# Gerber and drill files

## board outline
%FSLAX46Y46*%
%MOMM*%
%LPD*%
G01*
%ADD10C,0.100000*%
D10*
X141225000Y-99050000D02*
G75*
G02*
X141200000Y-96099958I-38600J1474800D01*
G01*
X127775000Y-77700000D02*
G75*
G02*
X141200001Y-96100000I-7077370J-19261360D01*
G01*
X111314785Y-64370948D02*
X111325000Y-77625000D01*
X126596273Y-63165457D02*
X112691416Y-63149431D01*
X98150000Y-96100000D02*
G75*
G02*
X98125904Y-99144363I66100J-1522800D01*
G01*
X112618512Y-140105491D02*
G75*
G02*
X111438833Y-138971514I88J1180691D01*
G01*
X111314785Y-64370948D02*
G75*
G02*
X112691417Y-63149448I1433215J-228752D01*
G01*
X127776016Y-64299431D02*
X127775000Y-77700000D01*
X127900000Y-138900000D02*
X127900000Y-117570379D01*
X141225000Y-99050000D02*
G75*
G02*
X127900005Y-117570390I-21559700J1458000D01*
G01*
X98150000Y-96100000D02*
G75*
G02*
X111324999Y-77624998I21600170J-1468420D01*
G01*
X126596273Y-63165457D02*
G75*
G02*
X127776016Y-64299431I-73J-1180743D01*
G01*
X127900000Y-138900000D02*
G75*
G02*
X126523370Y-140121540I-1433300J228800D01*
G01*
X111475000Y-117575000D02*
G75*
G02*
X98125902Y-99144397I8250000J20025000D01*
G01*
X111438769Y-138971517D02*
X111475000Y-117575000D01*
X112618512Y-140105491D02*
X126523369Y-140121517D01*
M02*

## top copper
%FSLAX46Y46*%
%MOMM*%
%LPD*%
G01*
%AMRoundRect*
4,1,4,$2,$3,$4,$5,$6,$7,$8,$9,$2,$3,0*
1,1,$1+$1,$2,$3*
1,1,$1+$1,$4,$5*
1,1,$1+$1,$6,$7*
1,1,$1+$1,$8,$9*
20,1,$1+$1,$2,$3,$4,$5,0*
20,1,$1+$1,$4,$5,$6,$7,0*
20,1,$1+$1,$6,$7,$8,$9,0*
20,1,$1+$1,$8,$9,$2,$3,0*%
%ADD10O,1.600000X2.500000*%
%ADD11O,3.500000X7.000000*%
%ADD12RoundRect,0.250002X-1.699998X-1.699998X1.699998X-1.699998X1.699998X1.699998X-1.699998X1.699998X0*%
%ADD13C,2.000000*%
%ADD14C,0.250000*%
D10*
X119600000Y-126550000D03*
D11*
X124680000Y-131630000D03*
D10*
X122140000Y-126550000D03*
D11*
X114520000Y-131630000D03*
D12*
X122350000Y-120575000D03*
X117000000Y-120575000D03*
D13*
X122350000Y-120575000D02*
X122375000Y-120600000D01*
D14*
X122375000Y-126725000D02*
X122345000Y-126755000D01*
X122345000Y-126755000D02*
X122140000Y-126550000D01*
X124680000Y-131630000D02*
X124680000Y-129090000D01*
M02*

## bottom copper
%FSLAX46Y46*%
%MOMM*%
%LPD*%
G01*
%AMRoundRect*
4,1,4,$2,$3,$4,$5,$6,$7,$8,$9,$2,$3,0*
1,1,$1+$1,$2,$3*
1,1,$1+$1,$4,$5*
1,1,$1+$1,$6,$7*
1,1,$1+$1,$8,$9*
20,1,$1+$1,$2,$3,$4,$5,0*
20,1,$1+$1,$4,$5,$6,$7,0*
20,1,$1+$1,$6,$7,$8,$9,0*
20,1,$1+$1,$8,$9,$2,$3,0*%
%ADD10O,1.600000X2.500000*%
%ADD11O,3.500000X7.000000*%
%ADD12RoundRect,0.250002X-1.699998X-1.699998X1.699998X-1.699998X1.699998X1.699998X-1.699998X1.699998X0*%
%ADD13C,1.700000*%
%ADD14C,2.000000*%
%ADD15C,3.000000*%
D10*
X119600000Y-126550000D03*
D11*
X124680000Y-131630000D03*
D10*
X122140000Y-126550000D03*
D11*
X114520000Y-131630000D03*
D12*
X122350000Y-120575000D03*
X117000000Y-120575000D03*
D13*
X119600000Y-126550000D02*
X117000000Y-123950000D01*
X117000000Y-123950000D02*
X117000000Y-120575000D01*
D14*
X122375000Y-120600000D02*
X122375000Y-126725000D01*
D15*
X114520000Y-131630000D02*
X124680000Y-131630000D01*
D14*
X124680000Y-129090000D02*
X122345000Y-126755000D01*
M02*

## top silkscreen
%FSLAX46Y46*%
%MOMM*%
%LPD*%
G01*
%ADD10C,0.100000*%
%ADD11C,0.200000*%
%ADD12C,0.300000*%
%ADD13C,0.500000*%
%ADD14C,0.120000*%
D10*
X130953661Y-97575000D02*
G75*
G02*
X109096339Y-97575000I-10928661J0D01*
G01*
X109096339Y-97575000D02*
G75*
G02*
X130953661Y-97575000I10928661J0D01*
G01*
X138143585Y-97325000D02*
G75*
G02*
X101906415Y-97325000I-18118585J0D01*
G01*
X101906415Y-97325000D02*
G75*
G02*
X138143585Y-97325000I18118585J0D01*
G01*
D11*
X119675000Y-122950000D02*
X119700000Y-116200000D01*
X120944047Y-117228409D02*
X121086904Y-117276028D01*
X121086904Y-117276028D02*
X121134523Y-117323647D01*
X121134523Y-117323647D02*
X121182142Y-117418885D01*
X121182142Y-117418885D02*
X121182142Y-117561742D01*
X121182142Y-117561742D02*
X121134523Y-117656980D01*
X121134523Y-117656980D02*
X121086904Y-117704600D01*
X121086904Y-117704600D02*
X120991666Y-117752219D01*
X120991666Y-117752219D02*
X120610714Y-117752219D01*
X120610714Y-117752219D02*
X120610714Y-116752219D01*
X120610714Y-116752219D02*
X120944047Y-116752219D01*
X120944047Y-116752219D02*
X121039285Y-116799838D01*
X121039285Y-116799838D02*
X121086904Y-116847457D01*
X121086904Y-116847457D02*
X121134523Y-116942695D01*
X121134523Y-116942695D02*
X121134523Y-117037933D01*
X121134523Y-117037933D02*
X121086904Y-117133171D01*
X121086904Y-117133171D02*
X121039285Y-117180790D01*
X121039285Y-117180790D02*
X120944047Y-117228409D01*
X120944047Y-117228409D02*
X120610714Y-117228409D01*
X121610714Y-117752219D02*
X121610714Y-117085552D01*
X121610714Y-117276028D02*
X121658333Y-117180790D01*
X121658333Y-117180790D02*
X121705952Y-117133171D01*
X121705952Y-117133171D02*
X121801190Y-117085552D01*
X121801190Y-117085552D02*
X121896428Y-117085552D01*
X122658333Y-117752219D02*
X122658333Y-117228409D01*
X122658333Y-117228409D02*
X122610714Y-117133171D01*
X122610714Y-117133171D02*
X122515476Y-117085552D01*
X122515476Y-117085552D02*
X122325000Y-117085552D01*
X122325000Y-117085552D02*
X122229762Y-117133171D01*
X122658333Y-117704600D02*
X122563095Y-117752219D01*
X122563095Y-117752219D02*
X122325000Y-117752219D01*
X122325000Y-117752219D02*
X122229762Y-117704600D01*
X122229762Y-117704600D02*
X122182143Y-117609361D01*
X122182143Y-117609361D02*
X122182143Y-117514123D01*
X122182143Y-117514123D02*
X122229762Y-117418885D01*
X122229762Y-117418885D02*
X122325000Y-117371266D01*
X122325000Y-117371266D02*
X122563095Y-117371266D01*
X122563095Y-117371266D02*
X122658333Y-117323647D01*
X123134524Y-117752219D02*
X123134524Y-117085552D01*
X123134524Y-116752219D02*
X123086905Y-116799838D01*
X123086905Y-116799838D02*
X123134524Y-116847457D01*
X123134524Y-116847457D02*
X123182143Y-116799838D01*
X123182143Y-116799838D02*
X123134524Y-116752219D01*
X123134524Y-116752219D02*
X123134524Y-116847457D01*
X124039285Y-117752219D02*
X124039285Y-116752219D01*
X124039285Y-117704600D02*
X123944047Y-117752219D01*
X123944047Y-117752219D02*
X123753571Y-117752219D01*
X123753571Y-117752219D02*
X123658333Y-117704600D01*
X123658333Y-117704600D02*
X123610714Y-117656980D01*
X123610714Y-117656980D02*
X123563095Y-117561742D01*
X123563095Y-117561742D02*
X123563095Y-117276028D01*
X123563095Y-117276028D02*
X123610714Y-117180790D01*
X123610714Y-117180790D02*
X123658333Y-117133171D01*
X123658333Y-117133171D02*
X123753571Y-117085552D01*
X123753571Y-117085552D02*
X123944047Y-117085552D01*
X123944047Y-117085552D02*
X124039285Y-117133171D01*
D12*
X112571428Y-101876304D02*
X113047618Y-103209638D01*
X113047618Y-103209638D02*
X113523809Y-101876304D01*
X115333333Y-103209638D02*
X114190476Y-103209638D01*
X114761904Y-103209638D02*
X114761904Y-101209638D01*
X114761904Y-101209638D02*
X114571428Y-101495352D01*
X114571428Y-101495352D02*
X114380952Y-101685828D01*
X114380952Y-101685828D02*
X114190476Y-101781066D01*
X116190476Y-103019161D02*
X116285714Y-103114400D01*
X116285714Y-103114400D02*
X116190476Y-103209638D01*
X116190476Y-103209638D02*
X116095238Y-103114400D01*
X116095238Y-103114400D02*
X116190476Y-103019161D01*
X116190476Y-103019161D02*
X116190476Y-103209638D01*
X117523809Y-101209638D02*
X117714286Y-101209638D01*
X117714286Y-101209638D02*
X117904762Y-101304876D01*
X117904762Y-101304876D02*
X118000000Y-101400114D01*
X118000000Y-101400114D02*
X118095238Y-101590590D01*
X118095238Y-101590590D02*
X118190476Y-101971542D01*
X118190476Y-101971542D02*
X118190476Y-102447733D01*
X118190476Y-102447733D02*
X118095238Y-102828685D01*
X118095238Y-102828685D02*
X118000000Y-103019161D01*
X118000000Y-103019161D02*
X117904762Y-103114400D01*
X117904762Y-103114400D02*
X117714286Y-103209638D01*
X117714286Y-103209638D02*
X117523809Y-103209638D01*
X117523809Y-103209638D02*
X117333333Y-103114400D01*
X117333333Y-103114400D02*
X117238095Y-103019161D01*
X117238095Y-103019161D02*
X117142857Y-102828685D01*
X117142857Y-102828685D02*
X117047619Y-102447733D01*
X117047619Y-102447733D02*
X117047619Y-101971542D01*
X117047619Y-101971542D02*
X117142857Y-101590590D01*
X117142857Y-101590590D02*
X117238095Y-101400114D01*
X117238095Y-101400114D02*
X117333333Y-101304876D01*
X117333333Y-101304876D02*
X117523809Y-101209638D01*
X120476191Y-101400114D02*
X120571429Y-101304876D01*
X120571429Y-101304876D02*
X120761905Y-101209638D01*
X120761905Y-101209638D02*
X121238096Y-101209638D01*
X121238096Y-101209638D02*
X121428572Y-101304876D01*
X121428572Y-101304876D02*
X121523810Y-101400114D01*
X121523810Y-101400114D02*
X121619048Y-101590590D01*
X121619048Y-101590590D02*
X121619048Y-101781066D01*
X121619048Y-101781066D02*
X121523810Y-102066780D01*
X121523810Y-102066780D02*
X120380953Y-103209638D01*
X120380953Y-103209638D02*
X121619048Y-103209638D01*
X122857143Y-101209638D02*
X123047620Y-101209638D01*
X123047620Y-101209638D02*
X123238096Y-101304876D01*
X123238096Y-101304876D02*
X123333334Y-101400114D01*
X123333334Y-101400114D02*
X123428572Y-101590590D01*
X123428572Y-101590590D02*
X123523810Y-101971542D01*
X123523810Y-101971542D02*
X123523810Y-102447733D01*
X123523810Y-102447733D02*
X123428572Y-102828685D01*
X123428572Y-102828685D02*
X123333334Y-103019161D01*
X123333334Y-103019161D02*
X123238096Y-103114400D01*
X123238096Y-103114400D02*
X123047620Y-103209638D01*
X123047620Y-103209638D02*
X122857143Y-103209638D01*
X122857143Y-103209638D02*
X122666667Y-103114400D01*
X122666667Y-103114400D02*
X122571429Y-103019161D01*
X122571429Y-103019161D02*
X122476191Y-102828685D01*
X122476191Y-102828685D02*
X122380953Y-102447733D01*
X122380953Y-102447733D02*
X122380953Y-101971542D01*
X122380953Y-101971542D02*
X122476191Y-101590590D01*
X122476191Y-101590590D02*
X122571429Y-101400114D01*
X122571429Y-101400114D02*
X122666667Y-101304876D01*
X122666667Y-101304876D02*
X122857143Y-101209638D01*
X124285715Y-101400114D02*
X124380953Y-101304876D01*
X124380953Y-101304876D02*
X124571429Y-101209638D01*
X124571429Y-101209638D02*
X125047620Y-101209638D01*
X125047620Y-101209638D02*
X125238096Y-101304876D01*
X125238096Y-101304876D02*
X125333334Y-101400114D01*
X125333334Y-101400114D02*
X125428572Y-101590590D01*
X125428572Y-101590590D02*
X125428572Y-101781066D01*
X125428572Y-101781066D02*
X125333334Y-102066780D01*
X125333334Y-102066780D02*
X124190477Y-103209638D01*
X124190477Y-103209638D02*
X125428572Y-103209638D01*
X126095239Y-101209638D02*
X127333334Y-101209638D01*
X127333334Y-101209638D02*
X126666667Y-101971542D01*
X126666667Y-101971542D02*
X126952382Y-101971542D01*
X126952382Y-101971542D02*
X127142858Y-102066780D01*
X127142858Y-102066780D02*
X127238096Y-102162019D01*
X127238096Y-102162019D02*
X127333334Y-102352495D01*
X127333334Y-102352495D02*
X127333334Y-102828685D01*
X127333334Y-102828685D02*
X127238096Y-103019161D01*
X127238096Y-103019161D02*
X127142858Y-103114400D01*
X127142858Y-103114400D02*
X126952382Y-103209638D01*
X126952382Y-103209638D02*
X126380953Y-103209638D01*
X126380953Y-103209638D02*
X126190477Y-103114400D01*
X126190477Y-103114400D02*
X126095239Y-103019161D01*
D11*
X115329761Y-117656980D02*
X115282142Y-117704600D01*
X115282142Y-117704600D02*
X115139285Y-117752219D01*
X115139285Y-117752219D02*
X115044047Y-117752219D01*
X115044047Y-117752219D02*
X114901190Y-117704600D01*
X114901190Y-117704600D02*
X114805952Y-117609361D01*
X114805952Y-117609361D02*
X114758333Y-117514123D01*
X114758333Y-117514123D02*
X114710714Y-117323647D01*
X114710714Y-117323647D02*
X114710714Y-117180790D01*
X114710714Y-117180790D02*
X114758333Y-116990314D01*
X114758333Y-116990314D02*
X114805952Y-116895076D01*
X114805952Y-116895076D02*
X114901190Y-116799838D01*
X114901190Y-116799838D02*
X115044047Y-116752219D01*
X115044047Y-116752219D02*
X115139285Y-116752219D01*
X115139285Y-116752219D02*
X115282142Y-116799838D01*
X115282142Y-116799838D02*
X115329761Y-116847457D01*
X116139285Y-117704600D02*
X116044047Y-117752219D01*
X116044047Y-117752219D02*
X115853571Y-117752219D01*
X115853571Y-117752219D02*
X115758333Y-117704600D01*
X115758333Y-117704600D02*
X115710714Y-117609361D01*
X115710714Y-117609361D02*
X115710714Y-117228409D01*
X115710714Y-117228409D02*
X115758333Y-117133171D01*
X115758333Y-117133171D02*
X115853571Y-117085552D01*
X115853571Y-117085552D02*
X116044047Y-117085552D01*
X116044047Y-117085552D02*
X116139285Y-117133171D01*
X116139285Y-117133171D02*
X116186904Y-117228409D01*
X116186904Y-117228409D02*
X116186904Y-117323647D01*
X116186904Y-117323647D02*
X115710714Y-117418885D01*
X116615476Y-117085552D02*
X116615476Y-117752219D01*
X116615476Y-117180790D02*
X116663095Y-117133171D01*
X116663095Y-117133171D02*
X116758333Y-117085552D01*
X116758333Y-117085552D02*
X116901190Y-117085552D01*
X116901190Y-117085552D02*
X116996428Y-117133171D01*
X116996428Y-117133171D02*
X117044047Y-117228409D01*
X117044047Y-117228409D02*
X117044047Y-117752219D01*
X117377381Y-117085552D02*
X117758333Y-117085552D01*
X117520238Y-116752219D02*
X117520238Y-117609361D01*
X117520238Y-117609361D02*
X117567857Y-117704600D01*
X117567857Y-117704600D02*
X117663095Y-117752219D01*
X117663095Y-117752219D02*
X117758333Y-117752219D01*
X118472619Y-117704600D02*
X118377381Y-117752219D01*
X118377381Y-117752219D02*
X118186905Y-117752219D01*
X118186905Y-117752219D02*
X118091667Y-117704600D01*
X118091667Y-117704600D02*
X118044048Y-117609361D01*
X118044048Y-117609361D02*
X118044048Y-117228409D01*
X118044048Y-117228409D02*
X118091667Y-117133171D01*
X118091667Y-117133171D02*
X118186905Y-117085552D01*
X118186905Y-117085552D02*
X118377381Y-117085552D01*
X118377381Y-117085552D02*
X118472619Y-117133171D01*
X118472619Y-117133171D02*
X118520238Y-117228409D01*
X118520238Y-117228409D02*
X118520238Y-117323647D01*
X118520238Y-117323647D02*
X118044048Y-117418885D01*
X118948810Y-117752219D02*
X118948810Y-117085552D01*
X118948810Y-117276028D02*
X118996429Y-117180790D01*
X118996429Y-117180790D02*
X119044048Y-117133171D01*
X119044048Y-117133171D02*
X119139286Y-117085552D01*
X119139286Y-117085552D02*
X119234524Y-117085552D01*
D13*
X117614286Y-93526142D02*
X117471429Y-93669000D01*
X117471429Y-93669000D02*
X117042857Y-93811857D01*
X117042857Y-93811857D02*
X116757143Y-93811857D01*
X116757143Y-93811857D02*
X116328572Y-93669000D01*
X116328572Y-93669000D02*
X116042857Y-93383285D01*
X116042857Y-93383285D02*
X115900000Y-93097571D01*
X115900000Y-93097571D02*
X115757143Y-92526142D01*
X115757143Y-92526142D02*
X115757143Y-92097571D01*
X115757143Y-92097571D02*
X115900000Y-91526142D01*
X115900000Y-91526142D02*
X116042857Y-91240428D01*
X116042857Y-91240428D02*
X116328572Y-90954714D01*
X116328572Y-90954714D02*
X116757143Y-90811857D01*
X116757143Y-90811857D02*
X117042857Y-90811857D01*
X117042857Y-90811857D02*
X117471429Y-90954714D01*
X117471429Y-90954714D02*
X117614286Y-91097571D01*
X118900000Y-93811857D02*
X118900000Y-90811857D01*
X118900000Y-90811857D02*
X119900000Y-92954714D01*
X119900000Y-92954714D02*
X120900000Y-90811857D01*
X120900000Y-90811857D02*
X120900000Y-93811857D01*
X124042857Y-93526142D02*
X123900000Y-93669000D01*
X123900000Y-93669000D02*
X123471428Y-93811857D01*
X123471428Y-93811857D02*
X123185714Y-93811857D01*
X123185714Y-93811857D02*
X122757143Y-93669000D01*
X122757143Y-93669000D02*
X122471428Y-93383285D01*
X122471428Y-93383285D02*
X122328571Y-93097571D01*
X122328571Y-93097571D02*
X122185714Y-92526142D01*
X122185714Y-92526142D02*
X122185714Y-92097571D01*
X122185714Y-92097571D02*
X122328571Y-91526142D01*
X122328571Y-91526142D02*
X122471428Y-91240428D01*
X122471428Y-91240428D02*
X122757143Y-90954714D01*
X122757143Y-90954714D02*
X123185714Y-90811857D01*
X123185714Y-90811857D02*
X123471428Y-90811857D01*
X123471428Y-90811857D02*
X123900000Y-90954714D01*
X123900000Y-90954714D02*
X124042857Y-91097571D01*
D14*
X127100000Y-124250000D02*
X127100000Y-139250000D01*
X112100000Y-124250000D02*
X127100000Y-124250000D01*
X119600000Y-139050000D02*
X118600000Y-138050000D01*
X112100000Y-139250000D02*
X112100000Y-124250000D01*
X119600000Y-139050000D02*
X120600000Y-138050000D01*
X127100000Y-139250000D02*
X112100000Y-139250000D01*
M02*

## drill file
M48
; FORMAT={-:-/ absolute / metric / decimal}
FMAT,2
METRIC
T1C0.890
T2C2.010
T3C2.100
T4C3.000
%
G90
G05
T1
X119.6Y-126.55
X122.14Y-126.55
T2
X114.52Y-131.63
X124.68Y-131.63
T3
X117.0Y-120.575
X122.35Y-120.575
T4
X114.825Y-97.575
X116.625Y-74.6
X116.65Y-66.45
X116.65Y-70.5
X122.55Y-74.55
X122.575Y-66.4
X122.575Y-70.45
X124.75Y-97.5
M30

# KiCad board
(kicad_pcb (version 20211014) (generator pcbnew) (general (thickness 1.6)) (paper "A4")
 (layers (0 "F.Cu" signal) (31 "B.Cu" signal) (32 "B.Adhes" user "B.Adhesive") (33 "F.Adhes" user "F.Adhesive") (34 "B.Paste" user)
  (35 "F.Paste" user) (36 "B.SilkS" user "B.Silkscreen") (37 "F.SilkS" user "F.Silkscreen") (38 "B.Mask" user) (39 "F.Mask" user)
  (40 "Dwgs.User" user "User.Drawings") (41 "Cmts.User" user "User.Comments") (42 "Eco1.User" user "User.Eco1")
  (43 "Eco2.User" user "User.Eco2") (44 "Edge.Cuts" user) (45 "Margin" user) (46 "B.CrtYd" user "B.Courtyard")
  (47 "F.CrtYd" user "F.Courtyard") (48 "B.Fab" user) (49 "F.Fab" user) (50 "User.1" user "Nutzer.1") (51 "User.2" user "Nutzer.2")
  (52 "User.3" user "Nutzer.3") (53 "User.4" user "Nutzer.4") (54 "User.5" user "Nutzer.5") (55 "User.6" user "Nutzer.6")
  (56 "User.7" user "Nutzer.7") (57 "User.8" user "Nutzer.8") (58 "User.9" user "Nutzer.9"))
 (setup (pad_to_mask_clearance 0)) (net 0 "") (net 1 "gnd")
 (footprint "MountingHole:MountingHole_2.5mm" (layer "F.Cu") (at 122.575 70.45)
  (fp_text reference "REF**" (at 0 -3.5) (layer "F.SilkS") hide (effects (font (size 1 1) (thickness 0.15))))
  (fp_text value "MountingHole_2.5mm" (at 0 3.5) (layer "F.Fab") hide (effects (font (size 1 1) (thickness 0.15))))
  (pad "" np_thru_hole circle (at 0 0) (size 3 3) (drill 3) (layers F&B.Cu *.Mask)))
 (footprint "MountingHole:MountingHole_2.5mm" (layer "F.Cu") (at 122.575 66.4)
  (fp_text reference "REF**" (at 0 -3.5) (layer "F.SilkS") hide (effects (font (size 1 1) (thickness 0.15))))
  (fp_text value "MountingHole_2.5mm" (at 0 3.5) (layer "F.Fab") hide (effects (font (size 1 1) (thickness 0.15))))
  (pad "" np_thru_hole circle (at 0 0) (size 3 3) (drill 3) (layers F&B.Cu *.Mask)))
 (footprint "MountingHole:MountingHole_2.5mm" (layer "F.Cu") (at 122.55 74.55)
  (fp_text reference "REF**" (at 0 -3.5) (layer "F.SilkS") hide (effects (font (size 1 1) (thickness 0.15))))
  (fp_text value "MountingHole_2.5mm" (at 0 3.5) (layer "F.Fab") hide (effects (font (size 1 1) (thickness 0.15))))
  (pad "" np_thru_hole circle (at 0 0) (size 3 3) (drill 3) (layers F&B.Cu *.Mask)))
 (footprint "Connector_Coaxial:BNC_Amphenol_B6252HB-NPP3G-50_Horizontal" (layer "F.Cu") (at 119.6 126.55 180)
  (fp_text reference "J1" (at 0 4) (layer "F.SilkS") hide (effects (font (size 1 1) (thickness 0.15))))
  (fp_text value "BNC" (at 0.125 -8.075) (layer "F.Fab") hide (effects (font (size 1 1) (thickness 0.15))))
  (fp_line (start -7.5 2.3) (end -7.5 -12.7) (layer "F.SilkS") (width 0.12))
  (fp_line (start 7.5 2.3) (end -7.5 2.3) (layer "F.SilkS") (width 0.12))
  (fp_line (start 0 -12.5) (end 1 -11.5) (layer "F.SilkS") (width 0.12))
  (fp_line (start 7.5 -12.7) (end 7.5 2.3) (layer "F.SilkS") (width 0.12))
  (fp_line (start 0 -12.5) (end -1 -11.5) (layer "F.SilkS") (width 0.12))
  (fp_line (start -7.5 -12.7) (end 7.5 -12.7) (layer "F.SilkS") (width 0.12))
  (pad "1" thru_hole oval (at 0 0 180) (size 1.6 2.5) (drill 0.89) (layers *.Cu *.Mask))
  (pad "2" thru_hole oval (at -5.08 -5.08 180) (size 3.5 7) (drill 2.01) (layers *.Cu *.Mask) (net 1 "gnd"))
  (pad "2" thru_hole oval (at -2.54 0 180) (size 1.6 2.5) (drill 0.89) (layers *.Cu *.Mask))
  (pad "2" thru_hole oval (at 5.08 -5.08 180) (size 3.5 7) (drill 2.01) (layers *.Cu *.Mask)))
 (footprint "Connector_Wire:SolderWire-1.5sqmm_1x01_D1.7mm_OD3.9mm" (layer "F.Cu") (at 122.35 120.575)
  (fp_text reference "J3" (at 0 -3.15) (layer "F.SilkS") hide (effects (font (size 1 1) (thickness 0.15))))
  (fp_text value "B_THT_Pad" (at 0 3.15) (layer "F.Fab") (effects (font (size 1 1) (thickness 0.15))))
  (pad "1" thru_hole roundrect (at 0 0) (size 3.9 3.9) (drill 2.1) (layers *.Cu *.Mask) (roundrect_rratio 0.06410307692) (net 1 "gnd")))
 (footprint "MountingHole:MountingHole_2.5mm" (layer "F.Cu") (at 116.625 74.6)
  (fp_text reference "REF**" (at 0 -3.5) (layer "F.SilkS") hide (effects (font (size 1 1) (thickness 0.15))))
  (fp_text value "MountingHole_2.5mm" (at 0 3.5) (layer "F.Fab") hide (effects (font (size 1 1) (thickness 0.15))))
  (pad "" np_thru_hole circle (at 0 0) (size 3 3) (drill 3) (layers F&B.Cu *.Mask)))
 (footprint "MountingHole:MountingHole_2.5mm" (layer "F.Cu") (at 116.65 66.45)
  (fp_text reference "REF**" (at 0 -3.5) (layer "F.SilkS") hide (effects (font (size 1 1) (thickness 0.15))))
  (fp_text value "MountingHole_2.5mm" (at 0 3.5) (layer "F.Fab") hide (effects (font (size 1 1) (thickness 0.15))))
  (pad "" np_thru_hole circle (at 0 0) (size 3 3) (drill 3) (layers F&B.Cu *.Mask)))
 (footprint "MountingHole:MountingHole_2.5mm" (layer "F.Cu") (at 116.65 70.5)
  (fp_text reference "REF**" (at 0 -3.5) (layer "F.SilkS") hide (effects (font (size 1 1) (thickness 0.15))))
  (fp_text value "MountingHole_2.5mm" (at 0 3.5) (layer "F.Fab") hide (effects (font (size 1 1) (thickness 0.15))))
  (pad "" np_thru_hole circle (at 0 0) (size 3 3) (drill 3) (layers F&B.Cu *.Mask)))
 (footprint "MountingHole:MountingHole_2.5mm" (layer "F.Cu") (at 114.825 97.575)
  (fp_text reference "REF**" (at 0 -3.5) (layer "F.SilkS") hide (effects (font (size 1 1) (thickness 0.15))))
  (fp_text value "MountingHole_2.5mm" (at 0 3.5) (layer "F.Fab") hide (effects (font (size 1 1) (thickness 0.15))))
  (pad "" np_thru_hole circle (at 0 0) (size 3 3) (drill 3) (layers F&B.Cu *.Mask)))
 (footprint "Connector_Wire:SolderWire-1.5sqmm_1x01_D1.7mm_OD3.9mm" (layer "F.Cu") (at 117 120.575)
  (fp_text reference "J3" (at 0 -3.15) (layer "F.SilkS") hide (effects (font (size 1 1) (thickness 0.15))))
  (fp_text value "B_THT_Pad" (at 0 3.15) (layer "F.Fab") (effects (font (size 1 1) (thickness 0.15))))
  (pad "1" thru_hole roundrect (at 0 0) (size 3.9 3.9) (drill 2.1) (layers *.Cu *.Mask) (roundrect_rratio 0.06410307692)))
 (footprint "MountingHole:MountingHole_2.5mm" (layer "F.Cu") (at 124.75 97.5)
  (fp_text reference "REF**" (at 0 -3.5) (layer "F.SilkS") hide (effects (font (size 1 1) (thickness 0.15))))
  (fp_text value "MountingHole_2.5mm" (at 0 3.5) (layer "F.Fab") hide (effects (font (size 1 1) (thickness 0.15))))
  (pad "" np_thru_hole circle (at 0 0) (size 3 3) (drill 3) (layers F&B.Cu *.Mask)))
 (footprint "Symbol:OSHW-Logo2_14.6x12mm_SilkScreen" (layer "B.Cu") (at 119.775 107.375 180)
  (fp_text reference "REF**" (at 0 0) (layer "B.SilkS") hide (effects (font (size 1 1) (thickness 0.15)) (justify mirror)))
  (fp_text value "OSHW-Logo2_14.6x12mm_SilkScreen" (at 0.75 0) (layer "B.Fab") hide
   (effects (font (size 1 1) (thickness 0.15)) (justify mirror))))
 (gr_circle (center 120.025 97.575) (end 130.953661 97.575) (layer "F.SilkS") (width 0.1) (fill none))
 (gr_circle (center 120.025 97.325) (end 138.143585 97.325) (layer "F.SilkS") (width 0.1) (fill none))
 (gr_line (start 119.675 122.95) (end 119.7 116.2) (layer "F.SilkS") (width 0.2))
 (gr_arc (start 141.225 99.05) (mid 139.711132 97.587723) (end 141.2 96.1) (layer "Edge.Cuts") (width 0.1))
 (gr_arc (start 127.775 77.7) (mid 137.274739 84.866376) (end 141.2 96.1) (layer "Edge.Cuts") (width 0.1))
 (gr_line (start 111.314785 64.370948) (end 111.325 77.625) (layer "Edge.Cuts") (width 0.1))
 (gr_line (start 126.596273 63.165457) (end 112.691416 63.149431) (layer "Edge.Cuts") (width 0.1))
 (gr_arc (start 98.15 96.1) (mid 99.740276 97.634881) (end 98.125902 99.144397) (layer "Edge.Cuts") (width 0.1))
 (gr_arc (start 112.618512 140.105491) (mid 111.800341 139.776018) (end 111.438769 138.971517) (layer "Edge.Cuts") (width 0.1))
 (gr_arc (start 111.314785 64.370948) (mid 111.784728 63.514087) (end 112.691416 63.149431) (layer "Edge.Cuts") (width 0.1))
 (gr_line (start 127.776016 64.299431) (end 127.775 77.7) (layer "Edge.Cuts") (width 0.1))
 (gr_line (start 127.9 138.9) (end 127.9 117.570379) (layer "Edge.Cuts") (width 0.1))
 (gr_arc (start 141.225 99.05) (mid 137.206047 110.212163) (end 127.9 117.570379) (layer "Edge.Cuts") (width 0.1))
 (gr_arc (start 98.15 96.1) (mid 102.12156 85.000379) (end 111.325 77.625) (layer "Edge.Cuts") (width 0.1))
 (gr_arc (start 126.596273 63.165457) (mid 127.414444 63.49493) (end 127.776016 64.299431) (layer "Edge.Cuts") (width 0.1))
 (gr_arc (start 127.9 138.9) (mid 127.43005 139.756853) (end 126.523369 140.121517) (layer "Edge.Cuts") (width 0.1))
 (gr_arc (start 111.475 117.575) (mid 102.18465 110.254297) (end 98.125902 99.144397) (layer "Edge.Cuts") (width 0.1))
 (gr_line (start 111.438769 138.971517) (end 111.475 117.575) (layer "Edge.Cuts") (width 0.1))
 (gr_line (start 112.618512 140.105491) (end 126.523369 140.121517) (layer "Edge.Cuts") (width 0.1))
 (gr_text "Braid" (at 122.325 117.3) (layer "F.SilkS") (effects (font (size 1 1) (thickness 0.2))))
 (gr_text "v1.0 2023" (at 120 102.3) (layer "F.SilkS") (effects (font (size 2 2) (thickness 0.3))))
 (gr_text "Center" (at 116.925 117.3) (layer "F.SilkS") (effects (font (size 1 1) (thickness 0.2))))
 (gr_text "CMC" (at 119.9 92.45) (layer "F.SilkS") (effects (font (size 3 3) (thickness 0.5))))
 (segment (start 119.6 126.55) (end 117 123.95) (width 1.7) (layer "B.Cu") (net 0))
 (segment (start 117 123.95) (end 117 120.575) (width 1.7) (layer "B.Cu") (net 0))
 (segment (start 122.35 120.575) (end 122.375 120.6) (width 2) (layer "F.Cu") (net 1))
 (segment (start 122.375 126.725) (end 122.345 126.755) (width 0.25) (layer "F.Cu") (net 1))
 (segment (start 122.345 126.755) (end 122.14 126.55) (width 0.25) (layer "F.Cu") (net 1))
 (segment (start 124.68 131.63) (end 124.68 129.09) (width 0.25) (layer "F.Cu") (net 1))
 (segment (start 122.375 120.6) (end 122.375 126.725) (width 2) (layer "B.Cu") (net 1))
 (segment (start 114.52 131.63) (end 124.68 131.63) (width 3) (layer "B.Cu") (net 1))
 (segment (start 124.68 129.09) (end 122.345 126.755) (width 2) (layer "B.Cu") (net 1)))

